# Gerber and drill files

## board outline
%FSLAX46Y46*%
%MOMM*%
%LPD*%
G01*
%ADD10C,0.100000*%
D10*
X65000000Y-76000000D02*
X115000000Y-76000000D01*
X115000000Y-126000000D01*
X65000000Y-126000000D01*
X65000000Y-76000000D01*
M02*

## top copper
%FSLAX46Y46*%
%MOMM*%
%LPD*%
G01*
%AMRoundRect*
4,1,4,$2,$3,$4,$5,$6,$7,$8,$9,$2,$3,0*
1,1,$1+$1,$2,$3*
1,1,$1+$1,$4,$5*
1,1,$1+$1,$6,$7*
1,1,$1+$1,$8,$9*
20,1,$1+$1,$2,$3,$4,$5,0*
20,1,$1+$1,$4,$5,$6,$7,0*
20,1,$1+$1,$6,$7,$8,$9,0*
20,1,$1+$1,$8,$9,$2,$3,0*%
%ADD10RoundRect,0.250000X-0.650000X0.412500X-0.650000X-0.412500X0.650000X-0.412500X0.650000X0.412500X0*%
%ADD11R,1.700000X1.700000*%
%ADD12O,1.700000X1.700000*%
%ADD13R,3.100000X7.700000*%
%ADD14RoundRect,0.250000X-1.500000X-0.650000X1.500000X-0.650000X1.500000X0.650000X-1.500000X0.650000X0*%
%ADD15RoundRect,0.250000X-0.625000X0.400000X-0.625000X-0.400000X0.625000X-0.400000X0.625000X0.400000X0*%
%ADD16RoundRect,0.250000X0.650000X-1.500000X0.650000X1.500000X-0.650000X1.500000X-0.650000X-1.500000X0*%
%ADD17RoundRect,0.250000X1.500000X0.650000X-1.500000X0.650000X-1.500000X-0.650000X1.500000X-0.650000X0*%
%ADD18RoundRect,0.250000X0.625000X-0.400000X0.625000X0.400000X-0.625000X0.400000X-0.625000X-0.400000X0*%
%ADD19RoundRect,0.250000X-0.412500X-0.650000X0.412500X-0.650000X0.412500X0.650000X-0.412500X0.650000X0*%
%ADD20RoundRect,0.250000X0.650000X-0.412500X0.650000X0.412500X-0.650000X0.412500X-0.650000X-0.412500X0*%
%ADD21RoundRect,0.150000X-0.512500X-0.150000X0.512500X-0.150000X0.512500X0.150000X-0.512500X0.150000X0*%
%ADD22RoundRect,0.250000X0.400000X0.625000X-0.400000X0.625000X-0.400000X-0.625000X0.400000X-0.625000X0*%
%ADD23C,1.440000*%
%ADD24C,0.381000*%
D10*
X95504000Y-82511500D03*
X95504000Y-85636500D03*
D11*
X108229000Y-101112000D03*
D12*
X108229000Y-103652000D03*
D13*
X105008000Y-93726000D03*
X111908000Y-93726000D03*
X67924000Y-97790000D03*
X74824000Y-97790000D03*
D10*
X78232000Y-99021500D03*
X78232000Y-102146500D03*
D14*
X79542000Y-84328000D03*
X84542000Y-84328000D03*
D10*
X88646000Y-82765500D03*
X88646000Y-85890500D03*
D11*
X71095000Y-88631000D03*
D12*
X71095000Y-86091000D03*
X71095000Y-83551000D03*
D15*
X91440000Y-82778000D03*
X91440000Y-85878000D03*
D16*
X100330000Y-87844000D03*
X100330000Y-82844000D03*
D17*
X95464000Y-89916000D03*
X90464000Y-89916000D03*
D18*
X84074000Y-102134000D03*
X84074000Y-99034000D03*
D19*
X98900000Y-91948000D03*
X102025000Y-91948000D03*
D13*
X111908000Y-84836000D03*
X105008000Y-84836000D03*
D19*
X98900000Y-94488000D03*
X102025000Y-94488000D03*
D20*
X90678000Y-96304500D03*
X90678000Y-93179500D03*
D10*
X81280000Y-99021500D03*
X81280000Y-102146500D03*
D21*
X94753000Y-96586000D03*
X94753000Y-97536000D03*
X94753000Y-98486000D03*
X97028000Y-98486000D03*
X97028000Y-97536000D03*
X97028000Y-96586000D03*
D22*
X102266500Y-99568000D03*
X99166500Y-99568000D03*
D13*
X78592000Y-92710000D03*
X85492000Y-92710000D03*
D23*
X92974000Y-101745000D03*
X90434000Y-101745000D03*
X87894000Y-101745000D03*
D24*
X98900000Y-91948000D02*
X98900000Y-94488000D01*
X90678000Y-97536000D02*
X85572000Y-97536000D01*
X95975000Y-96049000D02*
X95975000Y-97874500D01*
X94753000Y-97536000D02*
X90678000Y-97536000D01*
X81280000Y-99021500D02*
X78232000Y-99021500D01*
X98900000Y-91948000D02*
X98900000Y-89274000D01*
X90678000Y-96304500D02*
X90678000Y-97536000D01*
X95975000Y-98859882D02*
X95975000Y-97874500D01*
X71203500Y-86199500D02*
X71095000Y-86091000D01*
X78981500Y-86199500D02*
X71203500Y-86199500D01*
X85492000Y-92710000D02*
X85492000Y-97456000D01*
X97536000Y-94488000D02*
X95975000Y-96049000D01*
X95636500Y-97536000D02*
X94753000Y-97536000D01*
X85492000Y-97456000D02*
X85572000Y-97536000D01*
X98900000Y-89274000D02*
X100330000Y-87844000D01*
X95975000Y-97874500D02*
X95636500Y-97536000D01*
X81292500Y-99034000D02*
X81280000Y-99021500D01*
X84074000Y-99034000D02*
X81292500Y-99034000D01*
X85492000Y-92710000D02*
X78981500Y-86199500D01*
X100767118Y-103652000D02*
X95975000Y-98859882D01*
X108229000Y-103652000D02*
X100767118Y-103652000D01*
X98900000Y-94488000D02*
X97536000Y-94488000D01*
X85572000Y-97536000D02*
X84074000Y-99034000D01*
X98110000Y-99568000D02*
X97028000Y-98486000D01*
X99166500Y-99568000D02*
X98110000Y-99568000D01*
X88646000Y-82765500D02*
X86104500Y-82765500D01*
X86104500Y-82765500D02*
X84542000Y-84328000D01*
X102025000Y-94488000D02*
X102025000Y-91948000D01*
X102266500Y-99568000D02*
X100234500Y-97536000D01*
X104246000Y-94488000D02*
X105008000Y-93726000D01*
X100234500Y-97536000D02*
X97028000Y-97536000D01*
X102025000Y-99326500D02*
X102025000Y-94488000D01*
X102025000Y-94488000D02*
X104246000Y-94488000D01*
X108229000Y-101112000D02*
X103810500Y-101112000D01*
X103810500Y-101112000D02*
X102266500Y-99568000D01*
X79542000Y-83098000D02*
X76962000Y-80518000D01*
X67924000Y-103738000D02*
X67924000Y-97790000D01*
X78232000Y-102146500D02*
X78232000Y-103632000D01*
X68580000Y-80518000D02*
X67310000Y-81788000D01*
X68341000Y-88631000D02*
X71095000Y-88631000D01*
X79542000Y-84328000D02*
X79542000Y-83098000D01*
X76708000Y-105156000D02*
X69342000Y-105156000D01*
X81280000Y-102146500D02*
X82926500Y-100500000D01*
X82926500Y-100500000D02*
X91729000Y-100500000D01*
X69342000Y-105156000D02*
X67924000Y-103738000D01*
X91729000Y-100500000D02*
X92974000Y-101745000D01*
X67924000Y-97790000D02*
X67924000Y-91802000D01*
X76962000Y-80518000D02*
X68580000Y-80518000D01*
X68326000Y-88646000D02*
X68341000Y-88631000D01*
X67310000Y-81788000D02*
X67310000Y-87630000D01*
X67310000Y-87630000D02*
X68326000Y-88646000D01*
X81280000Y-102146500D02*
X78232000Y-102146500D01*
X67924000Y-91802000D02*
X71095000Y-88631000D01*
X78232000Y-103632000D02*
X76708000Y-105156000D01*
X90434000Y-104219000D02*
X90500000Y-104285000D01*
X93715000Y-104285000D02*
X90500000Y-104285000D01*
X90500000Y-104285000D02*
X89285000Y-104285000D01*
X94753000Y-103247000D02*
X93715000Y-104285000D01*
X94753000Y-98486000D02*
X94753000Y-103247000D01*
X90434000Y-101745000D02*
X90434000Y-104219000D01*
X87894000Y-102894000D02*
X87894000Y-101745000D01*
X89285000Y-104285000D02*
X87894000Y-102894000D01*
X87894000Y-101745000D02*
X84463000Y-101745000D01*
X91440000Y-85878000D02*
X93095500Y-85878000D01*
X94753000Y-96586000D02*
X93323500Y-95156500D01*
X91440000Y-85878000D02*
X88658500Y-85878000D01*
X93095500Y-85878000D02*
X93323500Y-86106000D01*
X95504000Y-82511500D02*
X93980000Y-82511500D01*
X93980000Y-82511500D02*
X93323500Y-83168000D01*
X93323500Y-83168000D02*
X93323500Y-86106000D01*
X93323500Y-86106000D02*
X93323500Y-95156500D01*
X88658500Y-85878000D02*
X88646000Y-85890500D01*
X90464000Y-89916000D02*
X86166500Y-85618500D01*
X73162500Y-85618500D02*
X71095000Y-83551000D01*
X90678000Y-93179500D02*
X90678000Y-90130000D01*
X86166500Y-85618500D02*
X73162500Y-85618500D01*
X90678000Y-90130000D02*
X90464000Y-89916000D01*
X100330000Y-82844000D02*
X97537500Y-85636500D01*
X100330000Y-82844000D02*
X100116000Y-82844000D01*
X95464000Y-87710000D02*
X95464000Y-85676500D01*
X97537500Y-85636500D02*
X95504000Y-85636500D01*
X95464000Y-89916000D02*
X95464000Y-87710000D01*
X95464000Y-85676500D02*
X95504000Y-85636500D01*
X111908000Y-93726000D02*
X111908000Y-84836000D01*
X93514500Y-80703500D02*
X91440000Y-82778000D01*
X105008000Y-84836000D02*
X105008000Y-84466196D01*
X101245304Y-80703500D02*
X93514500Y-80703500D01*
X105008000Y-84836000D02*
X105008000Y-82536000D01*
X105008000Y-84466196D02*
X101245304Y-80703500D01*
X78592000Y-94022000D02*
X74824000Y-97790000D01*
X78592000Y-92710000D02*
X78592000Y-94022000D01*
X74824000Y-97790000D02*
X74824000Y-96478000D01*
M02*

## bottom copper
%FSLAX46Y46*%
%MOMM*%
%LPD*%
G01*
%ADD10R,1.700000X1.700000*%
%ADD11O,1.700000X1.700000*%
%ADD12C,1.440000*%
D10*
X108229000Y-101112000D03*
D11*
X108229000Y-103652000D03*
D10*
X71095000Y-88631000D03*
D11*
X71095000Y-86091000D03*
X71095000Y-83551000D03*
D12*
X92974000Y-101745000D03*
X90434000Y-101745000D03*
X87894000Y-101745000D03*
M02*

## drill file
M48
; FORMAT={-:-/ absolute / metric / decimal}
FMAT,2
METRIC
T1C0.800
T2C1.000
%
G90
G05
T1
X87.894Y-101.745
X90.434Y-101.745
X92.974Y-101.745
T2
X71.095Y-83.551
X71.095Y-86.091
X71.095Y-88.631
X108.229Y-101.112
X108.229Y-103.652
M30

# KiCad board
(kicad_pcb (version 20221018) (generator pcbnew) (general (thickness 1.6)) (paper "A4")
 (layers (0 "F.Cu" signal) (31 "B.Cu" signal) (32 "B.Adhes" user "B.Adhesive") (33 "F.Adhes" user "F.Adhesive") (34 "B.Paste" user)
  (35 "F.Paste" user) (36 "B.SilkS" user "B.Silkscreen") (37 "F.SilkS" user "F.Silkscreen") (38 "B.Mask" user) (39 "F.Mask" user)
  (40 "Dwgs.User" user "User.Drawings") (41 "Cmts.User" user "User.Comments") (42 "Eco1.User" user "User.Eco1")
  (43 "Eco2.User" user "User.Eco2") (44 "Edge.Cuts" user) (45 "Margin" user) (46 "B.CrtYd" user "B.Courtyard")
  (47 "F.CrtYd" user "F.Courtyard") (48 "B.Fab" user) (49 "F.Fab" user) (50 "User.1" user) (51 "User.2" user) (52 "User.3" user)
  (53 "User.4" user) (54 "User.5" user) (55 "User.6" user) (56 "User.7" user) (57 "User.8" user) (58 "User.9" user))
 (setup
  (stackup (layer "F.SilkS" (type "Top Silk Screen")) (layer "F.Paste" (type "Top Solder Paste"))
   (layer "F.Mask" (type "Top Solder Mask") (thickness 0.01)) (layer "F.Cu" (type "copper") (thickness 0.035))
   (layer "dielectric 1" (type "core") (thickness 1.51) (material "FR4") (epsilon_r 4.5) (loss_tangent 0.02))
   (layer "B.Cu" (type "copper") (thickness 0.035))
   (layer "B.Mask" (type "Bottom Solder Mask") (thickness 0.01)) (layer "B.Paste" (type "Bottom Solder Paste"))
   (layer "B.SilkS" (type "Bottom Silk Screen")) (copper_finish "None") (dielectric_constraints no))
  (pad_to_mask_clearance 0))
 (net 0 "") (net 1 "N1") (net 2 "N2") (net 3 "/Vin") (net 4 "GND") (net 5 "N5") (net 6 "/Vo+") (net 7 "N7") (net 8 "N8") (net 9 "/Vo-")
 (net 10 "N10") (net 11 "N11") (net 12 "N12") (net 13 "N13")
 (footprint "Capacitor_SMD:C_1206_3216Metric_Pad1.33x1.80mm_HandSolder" (layer "F.Cu") (at 95.504 84.074 -90)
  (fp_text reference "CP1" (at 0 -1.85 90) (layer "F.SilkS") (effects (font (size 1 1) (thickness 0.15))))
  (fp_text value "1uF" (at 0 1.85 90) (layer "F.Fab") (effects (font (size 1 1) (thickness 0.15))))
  (pad "1" smd roundrect (at -1.5625 0 270) (size 1.325 1.8) (layers "F.Cu" "F.Paste" "F.Mask") (roundrect_rratio 0.188679) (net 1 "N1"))
  (pad "2" smd roundrect (at 1.5625 0 270) (size 1.325 1.8) (layers "F.Cu" "F.Paste" "F.Mask") (roundrect_rratio 0.188679) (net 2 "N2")))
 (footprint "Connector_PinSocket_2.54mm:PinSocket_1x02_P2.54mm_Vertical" (layer "F.Cu") (at 108.229 101.112)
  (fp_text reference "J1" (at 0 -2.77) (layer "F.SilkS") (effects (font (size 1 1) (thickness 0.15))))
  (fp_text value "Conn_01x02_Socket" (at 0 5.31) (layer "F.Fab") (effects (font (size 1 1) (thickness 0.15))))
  (pad "1" thru_hole rect (at 0 0) (size 1.7 1.7) (drill 1) (layers "*.Cu" "*.Mask") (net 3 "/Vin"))
  (pad "2" thru_hole oval (at 0 2.54) (size 1.7 1.7) (drill 1) (layers "*.Cu" "*.Mask") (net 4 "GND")))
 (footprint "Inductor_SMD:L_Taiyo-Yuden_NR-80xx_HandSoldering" (layer "F.Cu") (at 108.458 93.726)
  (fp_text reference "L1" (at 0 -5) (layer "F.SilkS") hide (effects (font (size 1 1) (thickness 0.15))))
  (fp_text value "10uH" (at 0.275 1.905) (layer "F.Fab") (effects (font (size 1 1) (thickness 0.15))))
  (pad "1" smd rect (at -3.45 0) (size 3.1 7.7) (layers "F.Cu" "F.Paste" "F.Mask") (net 3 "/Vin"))
  (pad "2" smd rect (at 3.45 0) (size 3.1 7.7) (layers "F.Cu" "F.Paste" "F.Mask") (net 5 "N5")))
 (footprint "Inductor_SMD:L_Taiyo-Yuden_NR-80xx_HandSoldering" (layer "F.Cu") (at 71.374 97.79)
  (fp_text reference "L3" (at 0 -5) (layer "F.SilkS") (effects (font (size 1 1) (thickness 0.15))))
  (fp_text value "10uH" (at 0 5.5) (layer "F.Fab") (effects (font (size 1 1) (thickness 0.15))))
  (pad "1" smd rect (at -3.45 0) (size 3.1 7.7) (layers "F.Cu" "F.Paste" "F.Mask") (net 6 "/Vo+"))
  (pad "2" smd rect (at 3.45 0) (size 3.1 7.7) (layers "F.Cu" "F.Paste" "F.Mask") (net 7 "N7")))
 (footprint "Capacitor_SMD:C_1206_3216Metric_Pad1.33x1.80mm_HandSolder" (layer "F.Cu") (at 78.232 100.584 -90)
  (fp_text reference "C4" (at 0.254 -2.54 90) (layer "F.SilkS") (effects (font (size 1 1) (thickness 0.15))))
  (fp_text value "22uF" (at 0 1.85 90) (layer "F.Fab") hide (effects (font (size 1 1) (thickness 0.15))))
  (pad "1" smd roundrect (at -1.5625 0 270) (size 1.325 1.8) (layers "F.Cu" "F.Paste" "F.Mask") (roundrect_rratio 0.188679) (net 4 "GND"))
  (pad "2" smd roundrect (at 1.5625 0 270) (size 1.325 1.8) (layers "F.Cu" "F.Paste" "F.Mask") (roundrect_rratio 0.188679) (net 6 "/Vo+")))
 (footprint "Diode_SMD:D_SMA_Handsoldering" (layer "F.Cu") (at 82.042 84.328)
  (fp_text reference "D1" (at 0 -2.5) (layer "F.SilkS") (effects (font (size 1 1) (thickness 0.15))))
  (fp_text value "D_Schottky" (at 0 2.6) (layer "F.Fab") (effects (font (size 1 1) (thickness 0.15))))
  (pad "1" smd roundrect (at -2.5 0) (size 3.5 1.8) (layers "F.Cu" "F.Paste" "F.Mask") (roundrect_rratio 0.1388888889) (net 6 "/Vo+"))
  (pad "2" smd roundrect (at 2.5 0) (size 3.5 1.8) (layers "F.Cu" "F.Paste" "F.Mask") (roundrect_rratio 0.1388888889) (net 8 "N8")))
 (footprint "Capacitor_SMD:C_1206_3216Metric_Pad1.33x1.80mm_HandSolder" (layer "F.Cu") (at 88.646 84.328 -90)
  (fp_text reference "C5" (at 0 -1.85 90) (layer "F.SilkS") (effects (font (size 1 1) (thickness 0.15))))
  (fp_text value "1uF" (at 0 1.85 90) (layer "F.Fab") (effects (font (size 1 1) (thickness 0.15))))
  (pad "1" smd roundrect (at -1.5625 0 270) (size 1.325 1.8) (layers "F.Cu" "F.Paste" "F.Mask") (roundrect_rratio 0.188679) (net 8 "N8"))
  (pad "2" smd roundrect (at 1.5625 0 270) (size 1.325 1.8) (layers "F.Cu" "F.Paste" "F.Mask") (roundrect_rratio 0.188679) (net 1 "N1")))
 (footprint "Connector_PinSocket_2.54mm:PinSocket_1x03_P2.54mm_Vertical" (layer "F.Cu") (at 71.095 88.631 180)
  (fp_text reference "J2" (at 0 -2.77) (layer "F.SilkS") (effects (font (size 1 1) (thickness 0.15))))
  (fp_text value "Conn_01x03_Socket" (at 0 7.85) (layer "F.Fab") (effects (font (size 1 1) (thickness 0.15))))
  (pad "1" thru_hole rect (at 0 0 180) (size 1.7 1.7) (drill 1) (layers "*.Cu" "*.Mask") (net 6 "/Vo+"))
  (pad "2" thru_hole oval (at 0 2.54 180) (size 1.7 1.7) (drill 1) (layers "*.Cu" "*.Mask") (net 4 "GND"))
  (pad "3" thru_hole oval (at 0 5.08 180) (size 1.7 1.7) (drill 1) (layers "*.Cu" "*.Mask") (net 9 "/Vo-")))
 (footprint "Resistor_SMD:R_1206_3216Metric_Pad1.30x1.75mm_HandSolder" (layer "F.Cu") (at 91.44 84.328 -90)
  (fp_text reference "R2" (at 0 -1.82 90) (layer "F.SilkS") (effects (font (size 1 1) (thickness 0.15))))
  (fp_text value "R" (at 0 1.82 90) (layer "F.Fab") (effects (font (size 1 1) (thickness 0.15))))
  (pad "1" smd roundrect (at -1.55 0 270) (size 1.3 1.75) (layers "F.Cu" "F.Paste" "F.Mask") (roundrect_rratio 0.192308) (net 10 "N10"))
  (pad "2" smd roundrect (at 1.55 0 270) (size 1.3 1.75) (layers "F.Cu" "F.Paste" "F.Mask") (roundrect_rratio 0.192308) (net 1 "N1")))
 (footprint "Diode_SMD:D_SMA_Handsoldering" (layer "F.Cu") (at 100.33 85.344 90)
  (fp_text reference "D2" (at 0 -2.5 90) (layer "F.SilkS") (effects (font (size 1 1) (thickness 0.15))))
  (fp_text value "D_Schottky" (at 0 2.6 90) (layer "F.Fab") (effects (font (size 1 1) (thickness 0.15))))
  (pad "1" smd roundrect (at -2.5 0 90) (size 3.5 1.8) (layers "F.Cu" "F.Paste" "F.Mask") (roundrect_rratio 0.1388888889) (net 4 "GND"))
  (pad "2" smd roundrect (at 2.5 0 90) (size 3.5 1.8) (layers "F.Cu" "F.Paste" "F.Mask") (roundrect_rratio 0.1388888889) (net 2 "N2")))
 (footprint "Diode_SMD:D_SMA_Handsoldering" (layer "F.Cu") (at 92.964 89.916 180)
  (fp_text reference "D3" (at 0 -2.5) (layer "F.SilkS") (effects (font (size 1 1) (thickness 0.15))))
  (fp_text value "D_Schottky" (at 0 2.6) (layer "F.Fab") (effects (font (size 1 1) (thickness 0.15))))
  (pad "1" smd roundrect (at -2.5 0 180) (size 3.5 1.8) (layers "F.Cu" "F.Paste" "F.Mask") (roundrect_rratio 0.1388888889) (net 2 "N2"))
  (pad "2" smd roundrect (at 2.5 0 180) (size 3.5 1.8) (layers "F.Cu" "F.Paste" "F.Mask") (roundrect_rratio 0.1388888889) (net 9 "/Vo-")))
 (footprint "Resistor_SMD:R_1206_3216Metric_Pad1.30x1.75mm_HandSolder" (layer "F.Cu") (at 84.074 100.584 90)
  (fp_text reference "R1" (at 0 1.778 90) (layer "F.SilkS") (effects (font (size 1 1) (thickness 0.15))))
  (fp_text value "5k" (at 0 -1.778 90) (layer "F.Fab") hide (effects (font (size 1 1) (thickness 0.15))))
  (pad "1" smd roundrect (at -1.55 0 90) (size 1.3 1.75) (layers "F.Cu" "F.Paste" "F.Mask") (roundrect_rratio 0.192308) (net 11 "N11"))
  (pad "2" smd roundrect (at 1.55 0 90) (size 1.3 1.75) (layers "F.Cu" "F.Paste" "F.Mask") (roundrect_rratio 0.192308) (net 4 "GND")))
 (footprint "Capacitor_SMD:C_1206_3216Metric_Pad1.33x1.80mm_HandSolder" (layer "F.Cu") (at 100.4625 91.948)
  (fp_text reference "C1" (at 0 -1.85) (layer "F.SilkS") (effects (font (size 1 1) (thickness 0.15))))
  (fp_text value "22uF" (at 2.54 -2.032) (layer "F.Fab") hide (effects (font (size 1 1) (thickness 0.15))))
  (pad "1" smd roundrect (at -1.5625 0) (size 1.325 1.8) (layers "F.Cu" "F.Paste" "F.Mask") (roundrect_rratio 0.188679) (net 4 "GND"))
  (pad "2" smd roundrect (at 1.5625 0) (size 1.325 1.8) (layers "F.Cu" "F.Paste" "F.Mask") (roundrect_rratio 0.188679) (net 3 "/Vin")))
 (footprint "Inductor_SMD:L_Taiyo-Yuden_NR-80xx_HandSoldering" (layer "F.Cu") (at 108.458 84.836 180)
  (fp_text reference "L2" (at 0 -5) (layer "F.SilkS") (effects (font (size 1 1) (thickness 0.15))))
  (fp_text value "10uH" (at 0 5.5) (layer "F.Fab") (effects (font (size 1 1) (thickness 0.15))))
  (pad "1" smd rect (at -3.45 0 180) (size 3.1 7.7) (layers "F.Cu" "F.Paste" "F.Mask") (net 5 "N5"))
  (pad "2" smd rect (at 3.45 0 180) (size 3.1 7.7) (layers "F.Cu" "F.Paste" "F.Mask") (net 10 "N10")))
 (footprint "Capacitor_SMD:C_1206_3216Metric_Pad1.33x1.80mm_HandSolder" (layer "F.Cu") (at 100.4625 94.488)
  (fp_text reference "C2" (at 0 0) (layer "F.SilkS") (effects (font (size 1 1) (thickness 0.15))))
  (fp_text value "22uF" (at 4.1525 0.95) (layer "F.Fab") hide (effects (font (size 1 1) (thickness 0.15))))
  (pad "1" smd roundrect (at -1.5625 0) (size 1.325 1.8) (layers "F.Cu" "F.Paste" "F.Mask") (roundrect_rratio 0.188679) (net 4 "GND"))
  (pad "2" smd roundrect (at 1.5625 0) (size 1.325 1.8) (layers "F.Cu" "F.Paste" "F.Mask") (roundrect_rratio 0.188679) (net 3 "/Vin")))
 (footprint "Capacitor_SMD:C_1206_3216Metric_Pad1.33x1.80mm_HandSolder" (layer "F.Cu") (at 90.678 94.742 90)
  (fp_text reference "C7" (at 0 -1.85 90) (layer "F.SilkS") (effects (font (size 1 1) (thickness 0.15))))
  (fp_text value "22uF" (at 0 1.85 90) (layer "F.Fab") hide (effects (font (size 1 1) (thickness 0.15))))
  (pad "1" smd roundrect (at -1.5625 0 90) (size 1.325 1.8) (layers "F.Cu" "F.Paste" "F.Mask") (roundrect_rratio 0.188679) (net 4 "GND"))
  (pad "2" smd roundrect (at 1.5625 0 90) (size 1.325 1.8) (layers "F.Cu" "F.Paste" "F.Mask") (roundrect_rratio 0.188679) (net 9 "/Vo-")))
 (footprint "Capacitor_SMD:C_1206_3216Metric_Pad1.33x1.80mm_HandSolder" (layer "F.Cu") (at 81.28 100.584 -90)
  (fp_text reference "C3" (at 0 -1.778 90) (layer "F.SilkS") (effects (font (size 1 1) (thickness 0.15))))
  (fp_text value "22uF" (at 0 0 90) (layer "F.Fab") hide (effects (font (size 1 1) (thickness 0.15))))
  (pad "1" smd roundrect (at -1.5625 0 270) (size 1.325 1.8) (layers "F.Cu" "F.Paste" "F.Mask") (roundrect_rratio 0.188679) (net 4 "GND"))
  (pad "2" smd roundrect (at 1.5625 0 270) (size 1.325 1.8) (layers "F.Cu" "F.Paste" "F.Mask") (roundrect_rratio 0.188679) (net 6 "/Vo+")))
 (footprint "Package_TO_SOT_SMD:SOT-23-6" (layer "F.Cu") (at 95.8905 97.536)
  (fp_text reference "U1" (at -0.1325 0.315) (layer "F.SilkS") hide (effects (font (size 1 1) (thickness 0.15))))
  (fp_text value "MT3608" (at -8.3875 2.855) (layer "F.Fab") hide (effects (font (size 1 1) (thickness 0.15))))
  (pad "1" smd roundrect (at -1.1375 -0.95) (size 1.325 0.6) (layers "F.Cu" "F.Paste" "F.Mask") (roundrect_rratio 0.25) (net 1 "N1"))
  (pad "2" smd roundrect (at -1.1375 0) (size 1.325 0.6) (layers "F.Cu" "F.Paste" "F.Mask") (roundrect_rratio 0.25) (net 4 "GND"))
  (pad "3" smd roundrect (at -1.1375 0.95) (size 1.325 0.6) (layers "F.Cu" "F.Paste" "F.Mask") (roundrect_rratio 0.25) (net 11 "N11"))
  (pad "4" smd roundrect (at 1.1375 0.95) (size 1.325 0.6) (layers "F.Cu" "F.Paste" "F.Mask") (roundrect_rratio 0.25) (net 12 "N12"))
  (pad "5" smd roundrect (at 1.1375 0) (size 1.325 0.6) (layers "F.Cu" "F.Paste" "F.Mask") (roundrect_rratio 0.25) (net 3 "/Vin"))
  (pad "6" smd roundrect (at 1.1375 -0.95) (size 1.325 0.6) (layers "F.Cu" "F.Paste" "F.Mask") (roundrect_rratio 0.25) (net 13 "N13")))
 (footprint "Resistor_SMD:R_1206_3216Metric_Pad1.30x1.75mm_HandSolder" (layer "F.Cu") (at 100.7165 99.568 180)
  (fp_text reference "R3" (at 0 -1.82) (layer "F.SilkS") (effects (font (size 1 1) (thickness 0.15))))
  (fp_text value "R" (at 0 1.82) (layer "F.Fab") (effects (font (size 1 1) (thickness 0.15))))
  (pad "1" smd roundrect (at -1.55 0 180) (size 1.3 1.75) (layers "F.Cu" "F.Paste" "F.Mask") (roundrect_rratio 0.192308) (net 3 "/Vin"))
  (pad "2" smd roundrect (at 1.55 0 180) (size 1.3 1.75) (layers "F.Cu" "F.Paste" "F.Mask") (roundrect_rratio 0.192308) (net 12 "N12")))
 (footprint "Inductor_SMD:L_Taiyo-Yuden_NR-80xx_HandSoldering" (layer "F.Cu") (at 82.042 92.71)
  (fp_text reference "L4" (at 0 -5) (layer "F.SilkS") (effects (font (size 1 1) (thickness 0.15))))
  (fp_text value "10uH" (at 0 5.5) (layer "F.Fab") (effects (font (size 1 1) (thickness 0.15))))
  (pad "1" smd rect (at -3.45 0) (size 3.1 7.7) (layers "F.Cu" "F.Paste" "F.Mask") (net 7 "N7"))
  (pad "2" smd rect (at 3.45 0) (size 3.1 7.7) (layers "F.Cu" "F.Paste" "F.Mask") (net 4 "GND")))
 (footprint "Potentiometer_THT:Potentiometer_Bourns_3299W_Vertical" (layer "F.Cu") (at 92.974 101.745)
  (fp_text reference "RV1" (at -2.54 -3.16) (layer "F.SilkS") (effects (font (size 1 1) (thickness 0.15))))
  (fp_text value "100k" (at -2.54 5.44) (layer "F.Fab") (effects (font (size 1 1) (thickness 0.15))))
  (pad "1" thru_hole circle (at 0 0) (size 1.44 1.44) (drill 0.8) (layers "*.Cu" "*.Mask") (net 6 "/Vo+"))
  (pad "2" thru_hole circle (at -2.54 0) (size 1.44 1.44) (drill 0.8) (layers "*.Cu" "*.Mask") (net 11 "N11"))
  (pad "3" thru_hole circle (at -5.08 0) (size 1.44 1.44) (drill 0.8) (layers "*.Cu" "*.Mask") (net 11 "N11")))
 (gr_rect (start 65 76) (end 115 126) (stroke (width 0.1) (type default)) (fill none) (layer "Edge.Cuts"))
 (segment (start 98.9 91.948) (end 98.9 94.488) (width 0.381) (layer "F.Cu") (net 4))
 (segment (start 90.678 97.536) (end 85.572 97.536) (width 0.381) (layer "F.Cu") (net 4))
 (segment (start 95.975 96.049) (end 95.975 97.8745) (width 0.381) (layer "F.Cu") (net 4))
 (segment (start 94.753 97.536) (end 90.678 97.536) (width 0.381) (layer "F.Cu") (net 4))
 (segment (start 81.28 99.0215) (end 78.232 99.0215) (width 0.381) (layer "F.Cu") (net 4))
 (segment (start 98.9 91.948) (end 98.9 89.274) (width 0.381) (layer "F.Cu") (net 4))
 (segment (start 90.678 96.3045) (end 90.678 97.536) (width 0.381) (layer "F.Cu") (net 4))
 (segment (start 95.975 98.859882) (end 95.975 97.8745) (width 0.381) (layer "F.Cu") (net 4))
 (segment (start 71.2035 86.1995) (end 71.095 86.091) (width 0.381) (layer "F.Cu") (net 4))
 (segment (start 78.9815 86.1995) (end 71.2035 86.1995) (width 0.381) (layer "F.Cu") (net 4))
 (segment (start 85.492 92.71) (end 85.492 97.456) (width 0.381) (layer "F.Cu") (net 4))
 (segment (start 97.536 94.488) (end 95.975 96.049) (width 0.381) (layer "F.Cu") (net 4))
 (segment (start 95.6365 97.536) (end 94.753 97.536) (width 0.381) (layer "F.Cu") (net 4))
 (segment (start 85.492 97.456) (end 85.572 97.536) (width 0.381) (layer "F.Cu") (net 4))
 (segment (start 98.9 89.274) (end 100.33 87.844) (width 0.381) (layer "F.Cu") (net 4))
 (segment (start 95.975 97.8745) (end 95.6365 97.536) (width 0.381) (layer "F.Cu") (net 4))
 (segment (start 81.2925 99.034) (end 81.28 99.0215) (width 0.381) (layer "F.Cu") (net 4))
 (segment (start 84.074 99.034) (end 81.2925 99.034) (width 0.381) (layer "F.Cu") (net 4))
 (segment (start 85.492 92.71) (end 78.9815 86.1995) (width 0.381) (layer "F.Cu") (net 4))
 (segment (start 100.767118 103.652) (end 95.975 98.859882) (width 0.381) (layer "F.Cu") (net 4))
 (segment (start 108.229 103.652) (end 100.767118 103.652) (width 0.381) (layer "F.Cu") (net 4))
 (segment (start 98.9 94.488) (end 97.536 94.488) (width 0.381) (layer "F.Cu") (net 4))
 (segment (start 85.572 97.536) (end 84.074 99.034) (width 0.381) (layer "F.Cu") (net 4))
 (segment (start 98.11 99.568) (end 97.028 98.486) (width 0.381) (layer "F.Cu") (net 12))
 (segment (start 99.1665 99.568) (end 98.11 99.568) (width 0.381) (layer "F.Cu") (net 12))
 (segment (start 88.646 82.7655) (end 86.1045 82.7655) (width 0.381) (layer "F.Cu") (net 8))
 (segment (start 86.1045 82.7655) (end 84.542 84.328) (width 0.381) (layer "F.Cu") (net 8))
 (segment (start 102.025 94.488) (end 102.025 91.948) (width 0.381) (layer "F.Cu") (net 3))
 (segment (start 102.2665 99.568) (end 100.2345 97.536) (width 0.381) (layer "F.Cu") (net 3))
 (segment (start 104.246 94.488) (end 105.008 93.726) (width 0.381) (layer "F.Cu") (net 3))
 (segment (start 100.2345 97.536) (end 97.028 97.536) (width 0.381) (layer "F.Cu") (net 3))
 (segment (start 102.025 99.3265) (end 102.025 94.488) (width 0.381) (layer "F.Cu") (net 3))
 (segment (start 102.025 94.488) (end 104.246 94.488) (width 0.381) (layer "F.Cu") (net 3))
 (segment (start 108.229 101.112) (end 103.8105 101.112) (width 0.381) (layer "F.Cu") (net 3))
 (segment (start 103.8105 101.112) (end 102.2665 99.568) (width 0.381) (layer "F.Cu") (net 3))
 (segment (start 79.542 83.098) (end 76.962 80.518) (width 0.381) (layer "F.Cu") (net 6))
 (segment (start 67.924 103.738) (end 67.924 97.79) (width 0.381) (layer "F.Cu") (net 6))
 (segment (start 78.232 102.1465) (end 78.232 103.632) (width 0.381) (layer "F.Cu") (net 6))
 (segment (start 68.58 80.518) (end 67.31 81.788) (width 0.381) (layer "F.Cu") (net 6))
 (segment (start 68.341 88.631) (end 71.095 88.631) (width 0.381) (layer "F.Cu") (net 6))
 (segment (start 79.542 84.328) (end 79.542 83.098) (width 0.381) (layer "F.Cu") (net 6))
 (segment (start 76.708 105.156) (end 69.342 105.156) (width 0.381) (layer "F.Cu") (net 6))
 (segment (start 81.28 102.1465) (end 82.9265 100.5) (width 0.381) (layer "F.Cu") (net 6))
 (segment (start 82.9265 100.5) (end 91.729 100.5) (width 0.381) (layer "F.Cu") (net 6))
 (segment (start 69.342 105.156) (end 67.924 103.738) (width 0.381) (layer "F.Cu") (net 6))
 (segment (start 91.729 100.5) (end 92.974 101.745) (width 0.381) (layer "F.Cu") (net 6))
 (segment (start 67.924 97.79) (end 67.924 91.802) (width 0.381) (layer "F.Cu") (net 6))
 (segment (start 76.962 80.518) (end 68.58 80.518) (width 0.381) (layer "F.Cu") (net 6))
 (segment (start 68.326 88.646) (end 68.341 88.631) (width 0.381) (layer "F.Cu") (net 6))
 (segment (start 67.31 81.788) (end 67.31 87.63) (width 0.381) (layer "F.Cu") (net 6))
 (segment (start 67.31 87.63) (end 68.326 88.646) (width 0.381) (layer "F.Cu") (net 6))
 (segment (start 81.28 102.1465) (end 78.232 102.1465) (width 0.381) (layer "F.Cu") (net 6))
 (segment (start 67.924 91.802) (end 71.095 88.631) (width 0.381) (layer "F.Cu") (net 6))
 (segment (start 78.232 103.632) (end 76.708 105.156) (width 0.381) (layer "F.Cu") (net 6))
 (segment (start 90.434 104.219) (end 90.5 104.285) (width 0.381) (layer "F.Cu") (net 11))
 (segment (start 93.715 104.285) (end 90.5 104.285) (width 0.381) (layer "F.Cu") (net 11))
 (segment (start 90.5 104.285) (end 89.285 104.285) (width 0.381) (layer "F.Cu") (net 11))
 (segment (start 94.753 103.247) (end 93.715 104.285) (width 0.381) (layer "F.Cu") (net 11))
 (segment (start 94.753 98.486) (end 94.753 103.247) (width 0.381) (layer "F.Cu") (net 11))
 (segment (start 90.434 101.745) (end 90.434 104.219) (width 0.381) (layer "F.Cu") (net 11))
 (segment (start 87.894 102.894) (end 87.894 101.745) (width 0.381) (layer "F.Cu") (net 11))
 (segment (start 89.285 104.285) (end 87.894 102.894) (width 0.381) (layer "F.Cu") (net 11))
 (segment (start 87.894 101.745) (end 84.463 101.745) (width 0.381) (layer "F.Cu") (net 11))
 (segment (start 91.44 85.878) (end 93.0955 85.878) (width 0.381) (layer "F.Cu") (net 1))
 (segment (start 94.753 96.586) (end 93.3235 95.1565) (width 0.381) (layer "F.Cu") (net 1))
 (segment (start 91.44 85.878) (end 88.6585 85.878) (width 0.381) (layer "F.Cu") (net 1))
 (segment (start 93.0955 85.878) (end 93.3235 86.106) (width 0.381) (layer "F.Cu") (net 1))
 (segment (start 95.504 82.5115) (end 93.98 82.5115) (width 0.381) (layer "F.Cu") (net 1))
 (segment (start 93.98 82.5115) (end 93.3235 83.168) (width 0.381) (layer "F.Cu") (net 1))
 (segment (start 93.3235 83.168) (end 93.3235 86.106) (width 0.381) (layer "F.Cu") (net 1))
 (segment (start 93.3235 86.106) (end 93.3235 95.1565) (width 0.381) (layer "F.Cu") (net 1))
 (segment (start 88.6585 85.878) (end 88.646 85.8905) (width 0.381) (layer "F.Cu") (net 1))
 (segment (start 90.464 89.916) (end 86.1665 85.6185) (width 0.381) (layer "F.Cu") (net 9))
 (segment (start 73.1625 85.6185) (end 71.095 83.551) (width 0.381) (layer "F.Cu") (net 9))
 (segment (start 90.678 93.1795) (end 90.678 90.13) (width 0.381) (layer "F.Cu") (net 9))
 (segment (start 86.1665 85.6185) (end 73.1625 85.6185) (width 0.381) (layer "F.Cu") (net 9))
 (segment (start 90.678 90.13) (end 90.464 89.916) (width 0.381) (layer "F.Cu") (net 9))
 (segment (start 100.33 82.844) (end 97.5375 85.6365) (width 0.381) (layer "F.Cu") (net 2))
 (segment (start 100.33 82.844) (end 100.116 82.844) (width 0.381) (layer "F.Cu") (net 2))
 (segment (start 95.464 87.71) (end 95.464 85.6765) (width 0.381) (layer "F.Cu") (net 2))
 (segment (start 97.5375 85.6365) (end 95.504 85.6365) (width 0.381) (layer "F.Cu") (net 2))
 (segment (start 95.464 89.916) (end 95.464 87.71) (width 0.381) (layer "F.Cu") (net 2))
 (segment (start 95.464 85.6765) (end 95.504 85.6365) (width 0.381) (layer "F.Cu") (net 2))
 (segment (start 111.908 93.726) (end 111.908 84.836) (width 0.381) (layer "F.Cu") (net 5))
 (segment (start 93.5145 80.7035) (end 91.44 82.778) (width 0.381) (layer "F.Cu") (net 10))
 (segment (start 105.008 84.836) (end 105.008 84.466196) (width 0.381) (layer "F.Cu") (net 10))
 (segment (start 101.245304 80.7035) (end 93.5145 80.7035) (width 0.381) (layer "F.Cu") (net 10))
 (segment (start 105.008 84.836) (end 105.008 82.536) (width 0.381) (layer "F.Cu") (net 10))
 (segment (start 105.008 84.466196) (end 101.245304 80.7035) (width 0.381) (layer "F.Cu") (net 10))
 (segment (start 78.592 94.022) (end 74.824 97.79) (width 0.381) (layer "F.Cu") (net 7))
 (segment (start 78.592 92.71) (end 78.592 94.022) (width 0.381) (layer "F.Cu") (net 7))
 (segment (start 74.824 97.79) (end 74.824 96.478) (width 0.381) (layer "F.Cu") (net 7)))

